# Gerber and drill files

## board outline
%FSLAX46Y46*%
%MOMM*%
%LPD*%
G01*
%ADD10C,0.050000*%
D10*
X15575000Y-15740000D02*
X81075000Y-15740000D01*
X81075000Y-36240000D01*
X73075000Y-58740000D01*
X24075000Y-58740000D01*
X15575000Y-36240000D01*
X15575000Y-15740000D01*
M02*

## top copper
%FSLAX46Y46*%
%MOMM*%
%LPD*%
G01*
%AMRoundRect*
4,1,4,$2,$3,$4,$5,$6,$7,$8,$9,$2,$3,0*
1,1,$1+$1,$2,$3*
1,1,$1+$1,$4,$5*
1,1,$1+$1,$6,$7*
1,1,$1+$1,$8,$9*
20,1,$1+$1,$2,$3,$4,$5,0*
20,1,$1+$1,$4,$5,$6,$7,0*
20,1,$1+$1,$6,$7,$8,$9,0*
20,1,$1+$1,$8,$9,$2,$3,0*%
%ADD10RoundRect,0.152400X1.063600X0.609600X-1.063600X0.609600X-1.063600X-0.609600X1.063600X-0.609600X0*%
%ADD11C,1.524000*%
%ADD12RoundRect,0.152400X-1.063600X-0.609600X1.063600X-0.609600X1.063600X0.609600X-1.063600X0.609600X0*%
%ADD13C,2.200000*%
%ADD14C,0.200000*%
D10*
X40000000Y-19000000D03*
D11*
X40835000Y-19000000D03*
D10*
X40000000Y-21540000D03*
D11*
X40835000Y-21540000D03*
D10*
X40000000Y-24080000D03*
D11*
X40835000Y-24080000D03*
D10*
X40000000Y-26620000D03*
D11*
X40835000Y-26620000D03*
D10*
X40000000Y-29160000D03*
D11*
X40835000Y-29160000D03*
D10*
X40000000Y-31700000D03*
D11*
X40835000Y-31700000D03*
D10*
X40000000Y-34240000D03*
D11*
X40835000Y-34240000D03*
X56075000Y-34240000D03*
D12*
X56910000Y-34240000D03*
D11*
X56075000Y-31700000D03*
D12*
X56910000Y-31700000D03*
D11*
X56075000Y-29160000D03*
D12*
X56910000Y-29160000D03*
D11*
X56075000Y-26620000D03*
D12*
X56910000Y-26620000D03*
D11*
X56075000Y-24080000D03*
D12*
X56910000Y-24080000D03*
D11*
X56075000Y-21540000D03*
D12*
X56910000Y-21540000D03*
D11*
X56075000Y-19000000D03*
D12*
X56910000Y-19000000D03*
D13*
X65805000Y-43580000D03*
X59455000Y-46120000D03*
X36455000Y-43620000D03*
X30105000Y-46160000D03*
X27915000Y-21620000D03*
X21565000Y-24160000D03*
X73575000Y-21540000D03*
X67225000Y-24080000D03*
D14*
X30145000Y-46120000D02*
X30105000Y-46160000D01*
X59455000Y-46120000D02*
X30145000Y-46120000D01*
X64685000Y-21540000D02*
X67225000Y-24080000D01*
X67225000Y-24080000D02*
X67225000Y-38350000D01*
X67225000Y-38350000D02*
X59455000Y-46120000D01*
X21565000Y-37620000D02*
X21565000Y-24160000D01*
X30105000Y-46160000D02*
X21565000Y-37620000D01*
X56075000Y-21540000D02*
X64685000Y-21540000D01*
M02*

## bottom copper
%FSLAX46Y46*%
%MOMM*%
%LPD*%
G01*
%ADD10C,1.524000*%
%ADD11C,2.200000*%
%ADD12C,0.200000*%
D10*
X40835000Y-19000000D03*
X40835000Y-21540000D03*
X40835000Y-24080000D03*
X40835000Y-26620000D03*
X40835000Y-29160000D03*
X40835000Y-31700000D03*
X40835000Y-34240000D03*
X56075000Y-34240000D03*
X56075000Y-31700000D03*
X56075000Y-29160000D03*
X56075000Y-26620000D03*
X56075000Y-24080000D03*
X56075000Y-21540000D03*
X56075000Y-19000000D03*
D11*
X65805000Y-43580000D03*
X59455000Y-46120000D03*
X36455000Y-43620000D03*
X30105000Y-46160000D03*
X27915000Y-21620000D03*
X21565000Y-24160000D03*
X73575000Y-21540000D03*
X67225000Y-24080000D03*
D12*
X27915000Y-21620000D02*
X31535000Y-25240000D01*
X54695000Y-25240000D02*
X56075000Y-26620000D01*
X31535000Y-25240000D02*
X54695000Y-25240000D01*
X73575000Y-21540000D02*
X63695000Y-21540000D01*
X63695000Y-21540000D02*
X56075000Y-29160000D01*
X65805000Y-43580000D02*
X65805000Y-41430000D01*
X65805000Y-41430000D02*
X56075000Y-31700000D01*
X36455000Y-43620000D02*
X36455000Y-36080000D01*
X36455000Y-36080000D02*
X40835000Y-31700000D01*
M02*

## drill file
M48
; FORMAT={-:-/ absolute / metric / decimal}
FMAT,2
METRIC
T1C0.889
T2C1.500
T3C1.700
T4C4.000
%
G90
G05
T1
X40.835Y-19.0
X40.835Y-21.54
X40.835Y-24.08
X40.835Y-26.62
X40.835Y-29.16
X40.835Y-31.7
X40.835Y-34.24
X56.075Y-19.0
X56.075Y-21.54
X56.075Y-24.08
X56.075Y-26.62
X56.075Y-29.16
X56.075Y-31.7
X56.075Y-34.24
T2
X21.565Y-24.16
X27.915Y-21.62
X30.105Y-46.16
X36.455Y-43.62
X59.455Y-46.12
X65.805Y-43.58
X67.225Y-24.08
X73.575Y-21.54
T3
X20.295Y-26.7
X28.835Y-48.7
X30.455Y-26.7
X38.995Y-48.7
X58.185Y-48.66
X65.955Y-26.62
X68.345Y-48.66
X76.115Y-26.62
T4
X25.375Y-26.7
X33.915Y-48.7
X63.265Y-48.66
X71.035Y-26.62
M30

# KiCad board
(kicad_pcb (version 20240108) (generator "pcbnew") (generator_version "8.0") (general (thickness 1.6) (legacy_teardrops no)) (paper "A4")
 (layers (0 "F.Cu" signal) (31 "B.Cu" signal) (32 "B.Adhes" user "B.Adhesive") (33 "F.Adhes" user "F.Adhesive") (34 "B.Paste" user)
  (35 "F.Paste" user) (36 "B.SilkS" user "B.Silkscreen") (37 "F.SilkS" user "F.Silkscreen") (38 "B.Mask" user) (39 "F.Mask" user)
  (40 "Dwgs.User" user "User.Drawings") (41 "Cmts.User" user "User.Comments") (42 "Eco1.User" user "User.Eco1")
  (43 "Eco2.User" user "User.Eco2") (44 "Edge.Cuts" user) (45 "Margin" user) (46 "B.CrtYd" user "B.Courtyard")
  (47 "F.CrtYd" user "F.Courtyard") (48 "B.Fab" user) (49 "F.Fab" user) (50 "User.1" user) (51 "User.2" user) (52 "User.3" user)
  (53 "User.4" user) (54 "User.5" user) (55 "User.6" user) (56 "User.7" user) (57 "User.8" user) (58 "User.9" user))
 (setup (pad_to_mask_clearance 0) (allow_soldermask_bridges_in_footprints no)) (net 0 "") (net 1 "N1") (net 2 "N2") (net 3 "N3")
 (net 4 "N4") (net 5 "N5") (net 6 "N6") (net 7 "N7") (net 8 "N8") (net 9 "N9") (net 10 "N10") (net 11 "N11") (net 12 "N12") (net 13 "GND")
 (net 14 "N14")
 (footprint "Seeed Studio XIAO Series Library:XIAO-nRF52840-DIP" (layer "F.Cu") (at 48.455 26.62)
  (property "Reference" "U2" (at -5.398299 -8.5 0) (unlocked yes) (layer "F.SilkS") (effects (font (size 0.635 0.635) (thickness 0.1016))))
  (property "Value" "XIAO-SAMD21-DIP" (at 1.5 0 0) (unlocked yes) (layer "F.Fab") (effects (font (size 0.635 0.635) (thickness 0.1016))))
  (pad "1" smd roundrect (at -8.455 -7.62 180) (size 2.432 1.524) (layers "F.Cu" "F.Mask") (roundrect_rratio 0.1) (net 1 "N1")
   (thermal_bridge_angle 45))
  (pad "1" thru_hole circle (at -7.62 -7.62 180) (size 1.524 1.524) (drill 0.889) (layers "*.Cu" "*.Mask") (remove_unused_layers no)
   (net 1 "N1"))
  (pad "2" smd roundrect (at -8.455 -5.08 180) (size 2.432 1.524) (layers "F.Cu" "F.Mask") (roundrect_rratio 0.1) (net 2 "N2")
   (thermal_bridge_angle 45))
  (pad "2" thru_hole circle (at -7.62 -5.08 180) (size 1.524 1.524) (drill 0.889) (layers "*.Cu" "*.Mask") (remove_unused_layers no)
   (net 2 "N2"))
  (pad "3" smd roundrect (at -8.455 -2.54 180) (size 2.432 1.524) (layers "F.Cu" "F.Mask") (roundrect_rratio 0.1) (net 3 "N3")
   (thermal_bridge_angle 45))
  (pad "3" thru_hole circle (at -7.62 -2.54 180) (size 1.524 1.524) (drill 0.889) (layers "*.Cu" "*.Mask") (remove_unused_layers no)
   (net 3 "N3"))
  (pad "4" smd roundrect (at -8.455 0 180) (size 2.432 1.524) (layers "F.Cu" "F.Mask") (roundrect_rratio 0.1) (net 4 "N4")
   (thermal_bridge_angle 45))
  (pad "4" thru_hole circle (at -7.62 0 180) (size 1.524 1.524) (drill 0.889) (layers "*.Cu" "*.Mask") (remove_unused_layers no)
   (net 4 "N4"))
  (pad "5" smd roundrect (at -8.455 2.54 180) (size 2.432 1.524) (layers "F.Cu" "F.Mask") (roundrect_rratio 0.1) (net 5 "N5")
   (thermal_bridge_angle 45))
  (pad "5" thru_hole circle (at -7.62 2.54 180) (size 1.524 1.524) (drill 0.889) (layers "*.Cu" "*.Mask") (remove_unused_layers no)
   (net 5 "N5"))
  (pad "6" smd roundrect (at -8.455 5.08 180) (size 2.432 1.524) (layers "F.Cu" "F.Mask") (roundrect_rratio 0.1) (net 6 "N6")
   (thermal_bridge_angle 45))
  (pad "6" thru_hole circle (at -7.62 5.08 180) (size 1.524 1.524) (drill 0.889) (layers "*.Cu" "*.Mask") (remove_unused_layers no)
   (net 6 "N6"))
  (pad "7" smd roundrect (at -8.455 7.62 180) (size 2.432 1.524) (layers "F.Cu" "F.Mask") (roundrect_rratio 0.1) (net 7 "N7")
   (thermal_bridge_angle 45))
  (pad "7" thru_hole circle (at -7.62 7.62 180) (size 1.524 1.524) (drill 0.889) (layers "*.Cu" "*.Mask") (remove_unused_layers no)
   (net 7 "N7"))
  (pad "8" thru_hole circle (at 7.62 7.62) (size 1.524 1.524) (drill 0.889) (layers "*.Cu" "*.Mask") (remove_unused_layers no) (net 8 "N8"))
  (pad "8" smd roundrect (at 8.455 7.62) (size 2.432 1.524) (layers "F.Cu" "F.Mask") (roundrect_rratio 0.1) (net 8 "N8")
   (thermal_bridge_angle 45))
  (pad "9" thru_hole circle (at 7.62 5.08) (size 1.524 1.524) (drill 0.889) (layers "*.Cu" "*.Mask") (remove_unused_layers no) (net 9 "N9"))
  (pad "9" smd roundrect (at 8.455 5.08) (size 2.432 1.524) (layers "F.Cu" "F.Mask") (roundrect_rratio 0.1) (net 9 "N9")
   (thermal_bridge_angle 45))
  (pad "10" thru_hole circle (at 7.62 2.54) (size 1.524 1.524) (drill 0.889) (layers "*.Cu" "*.Mask") (remove_unused_layers no)
   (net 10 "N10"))
  (pad "10" smd roundrect (at 8.455 2.54) (size 2.432 1.524) (layers "F.Cu" "F.Mask") (roundrect_rratio 0.1) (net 10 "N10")
   (thermal_bridge_angle 45))
  (pad "11" thru_hole circle (at 7.62 0) (size 1.524 1.524) (drill 0.889) (layers "*.Cu" "*.Mask") (remove_unused_layers no) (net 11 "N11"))
  (pad "11" smd roundrect (at 8.455 0) (size 2.432 1.524) (layers "F.Cu" "F.Mask") (roundrect_rratio 0.1) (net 11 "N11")
   (thermal_bridge_angle 45))
  (pad "12" thru_hole circle (at 7.62 -2.54) (size 1.524 1.524) (drill 0.889) (layers "*.Cu" "*.Mask") (remove_unused_layers no)
   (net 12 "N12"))
  (pad "12" smd roundrect (at 8.455 -2.54) (size 2.432 1.524) (layers "F.Cu" "F.Mask") (roundrect_rratio 0.1) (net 12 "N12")
   (thermal_bridge_angle 45))
  (pad "13" thru_hole circle (at 7.62 -5.08) (size 1.524 1.524) (drill 0.889) (layers "*.Cu" "*.Mask") (remove_unused_layers no)
   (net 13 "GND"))
  (pad "13" smd roundrect (at 8.455 -5.08) (size 2.432 1.524) (layers "F.Cu" "F.Mask") (roundrect_rratio 0.1) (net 13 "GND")
   (thermal_bridge_angle 45))
  (pad "14" thru_hole circle (at 7.62 -7.62) (size 1.524 1.524) (drill 0.889) (layers "*.Cu" "*.Mask") (remove_unused_layers no)
   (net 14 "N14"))
  (pad "14" smd roundrect (at 8.455 -7.62) (size 2.432 1.524) (layers "F.Cu" "F.Mask") (roundrect_rratio 0.1) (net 14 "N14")
   (thermal_bridge_angle 45)))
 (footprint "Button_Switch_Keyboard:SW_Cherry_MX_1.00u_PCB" (layer "F.Cu") (at 65.805 43.58)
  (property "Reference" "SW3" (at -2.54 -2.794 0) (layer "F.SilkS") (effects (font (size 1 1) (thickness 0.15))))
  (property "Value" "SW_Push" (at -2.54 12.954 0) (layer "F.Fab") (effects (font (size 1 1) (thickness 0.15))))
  (pad "" np_thru_hole circle (at -7.62 5.08) (size 1.7 1.7) (drill 1.7) (layers "*.Cu" "*.Mask"))
  (pad "" np_thru_hole circle (at -2.54 5.08) (size 4 4) (drill 4) (layers "*.Cu" "*.Mask"))
  (pad "" np_thru_hole circle (at 2.54 5.08) (size 1.7 1.7) (drill 1.7) (layers "*.Cu" "*.Mask"))
  (pad "1" thru_hole circle (at 0 0) (size 2.2 2.2) (drill 1.5) (layers "*.Cu" "*.Mask") (remove_unused_layers no) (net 9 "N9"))
  (pad "2" thru_hole circle (at -6.35 2.54) (size 2.2 2.2) (drill 1.5) (layers "*.Cu" "*.Mask") (remove_unused_layers no) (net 13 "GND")))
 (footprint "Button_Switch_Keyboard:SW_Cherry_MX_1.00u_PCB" (layer "F.Cu") (at 36.455 43.62)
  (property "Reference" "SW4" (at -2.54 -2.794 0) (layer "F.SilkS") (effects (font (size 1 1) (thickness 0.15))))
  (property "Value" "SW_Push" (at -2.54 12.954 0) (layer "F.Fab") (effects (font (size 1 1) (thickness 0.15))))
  (pad "" np_thru_hole circle (at -7.62 5.08) (size 1.7 1.7) (drill 1.7) (layers "*.Cu" "*.Mask"))
  (pad "" np_thru_hole circle (at -2.54 5.08) (size 4 4) (drill 4) (layers "*.Cu" "*.Mask"))
  (pad "" np_thru_hole circle (at 2.54 5.08) (size 1.7 1.7) (drill 1.7) (layers "*.Cu" "*.Mask"))
  (pad "1" thru_hole circle (at 0 0) (size 2.2 2.2) (drill 1.5) (layers "*.Cu" "*.Mask") (remove_unused_layers no) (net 6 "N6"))
  (pad "2" thru_hole circle (at -6.35 2.54) (size 2.2 2.2) (drill 1.5) (layers "*.Cu" "*.Mask") (remove_unused_layers no) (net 13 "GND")))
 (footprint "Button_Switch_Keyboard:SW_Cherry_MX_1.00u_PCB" (layer "F.Cu") (at 27.915 21.62)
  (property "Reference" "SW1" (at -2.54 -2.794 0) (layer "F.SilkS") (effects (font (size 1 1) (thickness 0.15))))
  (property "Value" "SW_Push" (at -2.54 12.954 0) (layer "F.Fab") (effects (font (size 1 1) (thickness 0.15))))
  (pad "" np_thru_hole circle (at -7.62 5.08) (size 1.7 1.7) (drill 1.7) (layers "*.Cu" "*.Mask"))
  (pad "" np_thru_hole circle (at -2.54 5.08) (size 4 4) (drill 4) (layers "*.Cu" "*.Mask"))
  (pad "" np_thru_hole circle (at 2.54 5.08) (size 1.7 1.7) (drill 1.7) (layers "*.Cu" "*.Mask"))
  (pad "1" thru_hole circle (at 0 0) (size 2.2 2.2) (drill 1.5) (layers "*.Cu" "*.Mask") (remove_unused_layers no) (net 11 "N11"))
  (pad "2" thru_hole circle (at -6.35 2.54) (size 2.2 2.2) (drill 1.5) (layers "*.Cu" "*.Mask") (remove_unused_layers no) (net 13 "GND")))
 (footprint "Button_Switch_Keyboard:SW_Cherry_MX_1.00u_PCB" (layer "F.Cu") (at 73.575 21.54)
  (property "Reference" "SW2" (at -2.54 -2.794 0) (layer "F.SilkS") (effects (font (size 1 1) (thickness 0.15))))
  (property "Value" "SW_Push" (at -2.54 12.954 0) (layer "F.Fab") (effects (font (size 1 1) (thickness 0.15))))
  (pad "" np_thru_hole circle (at -7.62 5.08) (size 1.7 1.7) (drill 1.7) (layers "*.Cu" "*.Mask"))
  (pad "" np_thru_hole circle (at -2.54 5.08) (size 4 4) (drill 4) (layers "*.Cu" "*.Mask"))
  (pad "" np_thru_hole circle (at 2.54 5.08) (size 1.7 1.7) (drill 1.7) (layers "*.Cu" "*.Mask"))
  (pad "1" thru_hole circle (at 0 0) (size 2.2 2.2) (drill 1.5) (layers "*.Cu" "*.Mask") (remove_unused_layers no) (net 10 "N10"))
  (pad "2" thru_hole circle (at -6.35 2.54) (size 2.2 2.2) (drill 1.5) (layers "*.Cu" "*.Mask") (remove_unused_layers no) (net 13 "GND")))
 (gr_poly
  (pts (xy 15.575 15.74) (xy 81.075 15.74) (xy 81.075 36.24) (xy 73.075 58.74) (xy 24.075 58.74) (xy 15.575 36.24))
  (stroke (width 0.05) (type solid)) (fill none) (layer "Edge.Cuts"))
 (segment (start 30.145 46.12) (end 30.105 46.16) (width 0.2) (layer "F.Cu") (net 13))
 (segment (start 59.455 46.12) (end 30.145 46.12) (width 0.2) (layer "F.Cu") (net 13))
 (segment (start 64.685 21.54) (end 67.225 24.08) (width 0.2) (layer "F.Cu") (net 13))
 (segment (start 67.225 24.08) (end 67.225 38.35) (width 0.2) (layer "F.Cu") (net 13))
 (segment (start 67.225 38.35) (end 59.455 46.12) (width 0.2) (layer "F.Cu") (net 13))
 (segment (start 21.565 37.62) (end 21.565 24.16) (width 0.2) (layer "F.Cu") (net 13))
 (segment (start 30.105 46.16) (end 21.565 37.62) (width 0.2) (layer "F.Cu") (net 13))
 (segment (start 56.075 21.54) (end 64.685 21.54) (width 0.2) (layer "F.Cu") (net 13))
 (segment (start 27.915 21.62) (end 31.535 25.24) (width 0.2) (layer "B.Cu") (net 11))
 (segment (start 54.695 25.24) (end 56.075 26.62) (width 0.2) (layer "B.Cu") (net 11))
 (segment (start 31.535 25.24) (end 54.695 25.24) (width 0.2) (layer "B.Cu") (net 11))
 (segment (start 73.575 21.54) (end 63.695 21.54) (width 0.2) (layer "B.Cu") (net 10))
 (segment (start 63.695 21.54) (end 56.075 29.16) (width 0.2) (layer "B.Cu") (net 10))
 (segment (start 65.805 43.58) (end 65.805 41.43) (width 0.2) (layer "B.Cu") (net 9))
 (segment (start 65.805 41.43) (end 56.075 31.7) (width 0.2) (layer "B.Cu") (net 9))
 (segment (start 36.455 43.62) (end 36.455 36.08) (width 0.2) (layer "B.Cu") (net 6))
 (segment (start 36.455 36.08) (end 40.835 31.7) (width 0.2) (layer "B.Cu") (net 6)))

